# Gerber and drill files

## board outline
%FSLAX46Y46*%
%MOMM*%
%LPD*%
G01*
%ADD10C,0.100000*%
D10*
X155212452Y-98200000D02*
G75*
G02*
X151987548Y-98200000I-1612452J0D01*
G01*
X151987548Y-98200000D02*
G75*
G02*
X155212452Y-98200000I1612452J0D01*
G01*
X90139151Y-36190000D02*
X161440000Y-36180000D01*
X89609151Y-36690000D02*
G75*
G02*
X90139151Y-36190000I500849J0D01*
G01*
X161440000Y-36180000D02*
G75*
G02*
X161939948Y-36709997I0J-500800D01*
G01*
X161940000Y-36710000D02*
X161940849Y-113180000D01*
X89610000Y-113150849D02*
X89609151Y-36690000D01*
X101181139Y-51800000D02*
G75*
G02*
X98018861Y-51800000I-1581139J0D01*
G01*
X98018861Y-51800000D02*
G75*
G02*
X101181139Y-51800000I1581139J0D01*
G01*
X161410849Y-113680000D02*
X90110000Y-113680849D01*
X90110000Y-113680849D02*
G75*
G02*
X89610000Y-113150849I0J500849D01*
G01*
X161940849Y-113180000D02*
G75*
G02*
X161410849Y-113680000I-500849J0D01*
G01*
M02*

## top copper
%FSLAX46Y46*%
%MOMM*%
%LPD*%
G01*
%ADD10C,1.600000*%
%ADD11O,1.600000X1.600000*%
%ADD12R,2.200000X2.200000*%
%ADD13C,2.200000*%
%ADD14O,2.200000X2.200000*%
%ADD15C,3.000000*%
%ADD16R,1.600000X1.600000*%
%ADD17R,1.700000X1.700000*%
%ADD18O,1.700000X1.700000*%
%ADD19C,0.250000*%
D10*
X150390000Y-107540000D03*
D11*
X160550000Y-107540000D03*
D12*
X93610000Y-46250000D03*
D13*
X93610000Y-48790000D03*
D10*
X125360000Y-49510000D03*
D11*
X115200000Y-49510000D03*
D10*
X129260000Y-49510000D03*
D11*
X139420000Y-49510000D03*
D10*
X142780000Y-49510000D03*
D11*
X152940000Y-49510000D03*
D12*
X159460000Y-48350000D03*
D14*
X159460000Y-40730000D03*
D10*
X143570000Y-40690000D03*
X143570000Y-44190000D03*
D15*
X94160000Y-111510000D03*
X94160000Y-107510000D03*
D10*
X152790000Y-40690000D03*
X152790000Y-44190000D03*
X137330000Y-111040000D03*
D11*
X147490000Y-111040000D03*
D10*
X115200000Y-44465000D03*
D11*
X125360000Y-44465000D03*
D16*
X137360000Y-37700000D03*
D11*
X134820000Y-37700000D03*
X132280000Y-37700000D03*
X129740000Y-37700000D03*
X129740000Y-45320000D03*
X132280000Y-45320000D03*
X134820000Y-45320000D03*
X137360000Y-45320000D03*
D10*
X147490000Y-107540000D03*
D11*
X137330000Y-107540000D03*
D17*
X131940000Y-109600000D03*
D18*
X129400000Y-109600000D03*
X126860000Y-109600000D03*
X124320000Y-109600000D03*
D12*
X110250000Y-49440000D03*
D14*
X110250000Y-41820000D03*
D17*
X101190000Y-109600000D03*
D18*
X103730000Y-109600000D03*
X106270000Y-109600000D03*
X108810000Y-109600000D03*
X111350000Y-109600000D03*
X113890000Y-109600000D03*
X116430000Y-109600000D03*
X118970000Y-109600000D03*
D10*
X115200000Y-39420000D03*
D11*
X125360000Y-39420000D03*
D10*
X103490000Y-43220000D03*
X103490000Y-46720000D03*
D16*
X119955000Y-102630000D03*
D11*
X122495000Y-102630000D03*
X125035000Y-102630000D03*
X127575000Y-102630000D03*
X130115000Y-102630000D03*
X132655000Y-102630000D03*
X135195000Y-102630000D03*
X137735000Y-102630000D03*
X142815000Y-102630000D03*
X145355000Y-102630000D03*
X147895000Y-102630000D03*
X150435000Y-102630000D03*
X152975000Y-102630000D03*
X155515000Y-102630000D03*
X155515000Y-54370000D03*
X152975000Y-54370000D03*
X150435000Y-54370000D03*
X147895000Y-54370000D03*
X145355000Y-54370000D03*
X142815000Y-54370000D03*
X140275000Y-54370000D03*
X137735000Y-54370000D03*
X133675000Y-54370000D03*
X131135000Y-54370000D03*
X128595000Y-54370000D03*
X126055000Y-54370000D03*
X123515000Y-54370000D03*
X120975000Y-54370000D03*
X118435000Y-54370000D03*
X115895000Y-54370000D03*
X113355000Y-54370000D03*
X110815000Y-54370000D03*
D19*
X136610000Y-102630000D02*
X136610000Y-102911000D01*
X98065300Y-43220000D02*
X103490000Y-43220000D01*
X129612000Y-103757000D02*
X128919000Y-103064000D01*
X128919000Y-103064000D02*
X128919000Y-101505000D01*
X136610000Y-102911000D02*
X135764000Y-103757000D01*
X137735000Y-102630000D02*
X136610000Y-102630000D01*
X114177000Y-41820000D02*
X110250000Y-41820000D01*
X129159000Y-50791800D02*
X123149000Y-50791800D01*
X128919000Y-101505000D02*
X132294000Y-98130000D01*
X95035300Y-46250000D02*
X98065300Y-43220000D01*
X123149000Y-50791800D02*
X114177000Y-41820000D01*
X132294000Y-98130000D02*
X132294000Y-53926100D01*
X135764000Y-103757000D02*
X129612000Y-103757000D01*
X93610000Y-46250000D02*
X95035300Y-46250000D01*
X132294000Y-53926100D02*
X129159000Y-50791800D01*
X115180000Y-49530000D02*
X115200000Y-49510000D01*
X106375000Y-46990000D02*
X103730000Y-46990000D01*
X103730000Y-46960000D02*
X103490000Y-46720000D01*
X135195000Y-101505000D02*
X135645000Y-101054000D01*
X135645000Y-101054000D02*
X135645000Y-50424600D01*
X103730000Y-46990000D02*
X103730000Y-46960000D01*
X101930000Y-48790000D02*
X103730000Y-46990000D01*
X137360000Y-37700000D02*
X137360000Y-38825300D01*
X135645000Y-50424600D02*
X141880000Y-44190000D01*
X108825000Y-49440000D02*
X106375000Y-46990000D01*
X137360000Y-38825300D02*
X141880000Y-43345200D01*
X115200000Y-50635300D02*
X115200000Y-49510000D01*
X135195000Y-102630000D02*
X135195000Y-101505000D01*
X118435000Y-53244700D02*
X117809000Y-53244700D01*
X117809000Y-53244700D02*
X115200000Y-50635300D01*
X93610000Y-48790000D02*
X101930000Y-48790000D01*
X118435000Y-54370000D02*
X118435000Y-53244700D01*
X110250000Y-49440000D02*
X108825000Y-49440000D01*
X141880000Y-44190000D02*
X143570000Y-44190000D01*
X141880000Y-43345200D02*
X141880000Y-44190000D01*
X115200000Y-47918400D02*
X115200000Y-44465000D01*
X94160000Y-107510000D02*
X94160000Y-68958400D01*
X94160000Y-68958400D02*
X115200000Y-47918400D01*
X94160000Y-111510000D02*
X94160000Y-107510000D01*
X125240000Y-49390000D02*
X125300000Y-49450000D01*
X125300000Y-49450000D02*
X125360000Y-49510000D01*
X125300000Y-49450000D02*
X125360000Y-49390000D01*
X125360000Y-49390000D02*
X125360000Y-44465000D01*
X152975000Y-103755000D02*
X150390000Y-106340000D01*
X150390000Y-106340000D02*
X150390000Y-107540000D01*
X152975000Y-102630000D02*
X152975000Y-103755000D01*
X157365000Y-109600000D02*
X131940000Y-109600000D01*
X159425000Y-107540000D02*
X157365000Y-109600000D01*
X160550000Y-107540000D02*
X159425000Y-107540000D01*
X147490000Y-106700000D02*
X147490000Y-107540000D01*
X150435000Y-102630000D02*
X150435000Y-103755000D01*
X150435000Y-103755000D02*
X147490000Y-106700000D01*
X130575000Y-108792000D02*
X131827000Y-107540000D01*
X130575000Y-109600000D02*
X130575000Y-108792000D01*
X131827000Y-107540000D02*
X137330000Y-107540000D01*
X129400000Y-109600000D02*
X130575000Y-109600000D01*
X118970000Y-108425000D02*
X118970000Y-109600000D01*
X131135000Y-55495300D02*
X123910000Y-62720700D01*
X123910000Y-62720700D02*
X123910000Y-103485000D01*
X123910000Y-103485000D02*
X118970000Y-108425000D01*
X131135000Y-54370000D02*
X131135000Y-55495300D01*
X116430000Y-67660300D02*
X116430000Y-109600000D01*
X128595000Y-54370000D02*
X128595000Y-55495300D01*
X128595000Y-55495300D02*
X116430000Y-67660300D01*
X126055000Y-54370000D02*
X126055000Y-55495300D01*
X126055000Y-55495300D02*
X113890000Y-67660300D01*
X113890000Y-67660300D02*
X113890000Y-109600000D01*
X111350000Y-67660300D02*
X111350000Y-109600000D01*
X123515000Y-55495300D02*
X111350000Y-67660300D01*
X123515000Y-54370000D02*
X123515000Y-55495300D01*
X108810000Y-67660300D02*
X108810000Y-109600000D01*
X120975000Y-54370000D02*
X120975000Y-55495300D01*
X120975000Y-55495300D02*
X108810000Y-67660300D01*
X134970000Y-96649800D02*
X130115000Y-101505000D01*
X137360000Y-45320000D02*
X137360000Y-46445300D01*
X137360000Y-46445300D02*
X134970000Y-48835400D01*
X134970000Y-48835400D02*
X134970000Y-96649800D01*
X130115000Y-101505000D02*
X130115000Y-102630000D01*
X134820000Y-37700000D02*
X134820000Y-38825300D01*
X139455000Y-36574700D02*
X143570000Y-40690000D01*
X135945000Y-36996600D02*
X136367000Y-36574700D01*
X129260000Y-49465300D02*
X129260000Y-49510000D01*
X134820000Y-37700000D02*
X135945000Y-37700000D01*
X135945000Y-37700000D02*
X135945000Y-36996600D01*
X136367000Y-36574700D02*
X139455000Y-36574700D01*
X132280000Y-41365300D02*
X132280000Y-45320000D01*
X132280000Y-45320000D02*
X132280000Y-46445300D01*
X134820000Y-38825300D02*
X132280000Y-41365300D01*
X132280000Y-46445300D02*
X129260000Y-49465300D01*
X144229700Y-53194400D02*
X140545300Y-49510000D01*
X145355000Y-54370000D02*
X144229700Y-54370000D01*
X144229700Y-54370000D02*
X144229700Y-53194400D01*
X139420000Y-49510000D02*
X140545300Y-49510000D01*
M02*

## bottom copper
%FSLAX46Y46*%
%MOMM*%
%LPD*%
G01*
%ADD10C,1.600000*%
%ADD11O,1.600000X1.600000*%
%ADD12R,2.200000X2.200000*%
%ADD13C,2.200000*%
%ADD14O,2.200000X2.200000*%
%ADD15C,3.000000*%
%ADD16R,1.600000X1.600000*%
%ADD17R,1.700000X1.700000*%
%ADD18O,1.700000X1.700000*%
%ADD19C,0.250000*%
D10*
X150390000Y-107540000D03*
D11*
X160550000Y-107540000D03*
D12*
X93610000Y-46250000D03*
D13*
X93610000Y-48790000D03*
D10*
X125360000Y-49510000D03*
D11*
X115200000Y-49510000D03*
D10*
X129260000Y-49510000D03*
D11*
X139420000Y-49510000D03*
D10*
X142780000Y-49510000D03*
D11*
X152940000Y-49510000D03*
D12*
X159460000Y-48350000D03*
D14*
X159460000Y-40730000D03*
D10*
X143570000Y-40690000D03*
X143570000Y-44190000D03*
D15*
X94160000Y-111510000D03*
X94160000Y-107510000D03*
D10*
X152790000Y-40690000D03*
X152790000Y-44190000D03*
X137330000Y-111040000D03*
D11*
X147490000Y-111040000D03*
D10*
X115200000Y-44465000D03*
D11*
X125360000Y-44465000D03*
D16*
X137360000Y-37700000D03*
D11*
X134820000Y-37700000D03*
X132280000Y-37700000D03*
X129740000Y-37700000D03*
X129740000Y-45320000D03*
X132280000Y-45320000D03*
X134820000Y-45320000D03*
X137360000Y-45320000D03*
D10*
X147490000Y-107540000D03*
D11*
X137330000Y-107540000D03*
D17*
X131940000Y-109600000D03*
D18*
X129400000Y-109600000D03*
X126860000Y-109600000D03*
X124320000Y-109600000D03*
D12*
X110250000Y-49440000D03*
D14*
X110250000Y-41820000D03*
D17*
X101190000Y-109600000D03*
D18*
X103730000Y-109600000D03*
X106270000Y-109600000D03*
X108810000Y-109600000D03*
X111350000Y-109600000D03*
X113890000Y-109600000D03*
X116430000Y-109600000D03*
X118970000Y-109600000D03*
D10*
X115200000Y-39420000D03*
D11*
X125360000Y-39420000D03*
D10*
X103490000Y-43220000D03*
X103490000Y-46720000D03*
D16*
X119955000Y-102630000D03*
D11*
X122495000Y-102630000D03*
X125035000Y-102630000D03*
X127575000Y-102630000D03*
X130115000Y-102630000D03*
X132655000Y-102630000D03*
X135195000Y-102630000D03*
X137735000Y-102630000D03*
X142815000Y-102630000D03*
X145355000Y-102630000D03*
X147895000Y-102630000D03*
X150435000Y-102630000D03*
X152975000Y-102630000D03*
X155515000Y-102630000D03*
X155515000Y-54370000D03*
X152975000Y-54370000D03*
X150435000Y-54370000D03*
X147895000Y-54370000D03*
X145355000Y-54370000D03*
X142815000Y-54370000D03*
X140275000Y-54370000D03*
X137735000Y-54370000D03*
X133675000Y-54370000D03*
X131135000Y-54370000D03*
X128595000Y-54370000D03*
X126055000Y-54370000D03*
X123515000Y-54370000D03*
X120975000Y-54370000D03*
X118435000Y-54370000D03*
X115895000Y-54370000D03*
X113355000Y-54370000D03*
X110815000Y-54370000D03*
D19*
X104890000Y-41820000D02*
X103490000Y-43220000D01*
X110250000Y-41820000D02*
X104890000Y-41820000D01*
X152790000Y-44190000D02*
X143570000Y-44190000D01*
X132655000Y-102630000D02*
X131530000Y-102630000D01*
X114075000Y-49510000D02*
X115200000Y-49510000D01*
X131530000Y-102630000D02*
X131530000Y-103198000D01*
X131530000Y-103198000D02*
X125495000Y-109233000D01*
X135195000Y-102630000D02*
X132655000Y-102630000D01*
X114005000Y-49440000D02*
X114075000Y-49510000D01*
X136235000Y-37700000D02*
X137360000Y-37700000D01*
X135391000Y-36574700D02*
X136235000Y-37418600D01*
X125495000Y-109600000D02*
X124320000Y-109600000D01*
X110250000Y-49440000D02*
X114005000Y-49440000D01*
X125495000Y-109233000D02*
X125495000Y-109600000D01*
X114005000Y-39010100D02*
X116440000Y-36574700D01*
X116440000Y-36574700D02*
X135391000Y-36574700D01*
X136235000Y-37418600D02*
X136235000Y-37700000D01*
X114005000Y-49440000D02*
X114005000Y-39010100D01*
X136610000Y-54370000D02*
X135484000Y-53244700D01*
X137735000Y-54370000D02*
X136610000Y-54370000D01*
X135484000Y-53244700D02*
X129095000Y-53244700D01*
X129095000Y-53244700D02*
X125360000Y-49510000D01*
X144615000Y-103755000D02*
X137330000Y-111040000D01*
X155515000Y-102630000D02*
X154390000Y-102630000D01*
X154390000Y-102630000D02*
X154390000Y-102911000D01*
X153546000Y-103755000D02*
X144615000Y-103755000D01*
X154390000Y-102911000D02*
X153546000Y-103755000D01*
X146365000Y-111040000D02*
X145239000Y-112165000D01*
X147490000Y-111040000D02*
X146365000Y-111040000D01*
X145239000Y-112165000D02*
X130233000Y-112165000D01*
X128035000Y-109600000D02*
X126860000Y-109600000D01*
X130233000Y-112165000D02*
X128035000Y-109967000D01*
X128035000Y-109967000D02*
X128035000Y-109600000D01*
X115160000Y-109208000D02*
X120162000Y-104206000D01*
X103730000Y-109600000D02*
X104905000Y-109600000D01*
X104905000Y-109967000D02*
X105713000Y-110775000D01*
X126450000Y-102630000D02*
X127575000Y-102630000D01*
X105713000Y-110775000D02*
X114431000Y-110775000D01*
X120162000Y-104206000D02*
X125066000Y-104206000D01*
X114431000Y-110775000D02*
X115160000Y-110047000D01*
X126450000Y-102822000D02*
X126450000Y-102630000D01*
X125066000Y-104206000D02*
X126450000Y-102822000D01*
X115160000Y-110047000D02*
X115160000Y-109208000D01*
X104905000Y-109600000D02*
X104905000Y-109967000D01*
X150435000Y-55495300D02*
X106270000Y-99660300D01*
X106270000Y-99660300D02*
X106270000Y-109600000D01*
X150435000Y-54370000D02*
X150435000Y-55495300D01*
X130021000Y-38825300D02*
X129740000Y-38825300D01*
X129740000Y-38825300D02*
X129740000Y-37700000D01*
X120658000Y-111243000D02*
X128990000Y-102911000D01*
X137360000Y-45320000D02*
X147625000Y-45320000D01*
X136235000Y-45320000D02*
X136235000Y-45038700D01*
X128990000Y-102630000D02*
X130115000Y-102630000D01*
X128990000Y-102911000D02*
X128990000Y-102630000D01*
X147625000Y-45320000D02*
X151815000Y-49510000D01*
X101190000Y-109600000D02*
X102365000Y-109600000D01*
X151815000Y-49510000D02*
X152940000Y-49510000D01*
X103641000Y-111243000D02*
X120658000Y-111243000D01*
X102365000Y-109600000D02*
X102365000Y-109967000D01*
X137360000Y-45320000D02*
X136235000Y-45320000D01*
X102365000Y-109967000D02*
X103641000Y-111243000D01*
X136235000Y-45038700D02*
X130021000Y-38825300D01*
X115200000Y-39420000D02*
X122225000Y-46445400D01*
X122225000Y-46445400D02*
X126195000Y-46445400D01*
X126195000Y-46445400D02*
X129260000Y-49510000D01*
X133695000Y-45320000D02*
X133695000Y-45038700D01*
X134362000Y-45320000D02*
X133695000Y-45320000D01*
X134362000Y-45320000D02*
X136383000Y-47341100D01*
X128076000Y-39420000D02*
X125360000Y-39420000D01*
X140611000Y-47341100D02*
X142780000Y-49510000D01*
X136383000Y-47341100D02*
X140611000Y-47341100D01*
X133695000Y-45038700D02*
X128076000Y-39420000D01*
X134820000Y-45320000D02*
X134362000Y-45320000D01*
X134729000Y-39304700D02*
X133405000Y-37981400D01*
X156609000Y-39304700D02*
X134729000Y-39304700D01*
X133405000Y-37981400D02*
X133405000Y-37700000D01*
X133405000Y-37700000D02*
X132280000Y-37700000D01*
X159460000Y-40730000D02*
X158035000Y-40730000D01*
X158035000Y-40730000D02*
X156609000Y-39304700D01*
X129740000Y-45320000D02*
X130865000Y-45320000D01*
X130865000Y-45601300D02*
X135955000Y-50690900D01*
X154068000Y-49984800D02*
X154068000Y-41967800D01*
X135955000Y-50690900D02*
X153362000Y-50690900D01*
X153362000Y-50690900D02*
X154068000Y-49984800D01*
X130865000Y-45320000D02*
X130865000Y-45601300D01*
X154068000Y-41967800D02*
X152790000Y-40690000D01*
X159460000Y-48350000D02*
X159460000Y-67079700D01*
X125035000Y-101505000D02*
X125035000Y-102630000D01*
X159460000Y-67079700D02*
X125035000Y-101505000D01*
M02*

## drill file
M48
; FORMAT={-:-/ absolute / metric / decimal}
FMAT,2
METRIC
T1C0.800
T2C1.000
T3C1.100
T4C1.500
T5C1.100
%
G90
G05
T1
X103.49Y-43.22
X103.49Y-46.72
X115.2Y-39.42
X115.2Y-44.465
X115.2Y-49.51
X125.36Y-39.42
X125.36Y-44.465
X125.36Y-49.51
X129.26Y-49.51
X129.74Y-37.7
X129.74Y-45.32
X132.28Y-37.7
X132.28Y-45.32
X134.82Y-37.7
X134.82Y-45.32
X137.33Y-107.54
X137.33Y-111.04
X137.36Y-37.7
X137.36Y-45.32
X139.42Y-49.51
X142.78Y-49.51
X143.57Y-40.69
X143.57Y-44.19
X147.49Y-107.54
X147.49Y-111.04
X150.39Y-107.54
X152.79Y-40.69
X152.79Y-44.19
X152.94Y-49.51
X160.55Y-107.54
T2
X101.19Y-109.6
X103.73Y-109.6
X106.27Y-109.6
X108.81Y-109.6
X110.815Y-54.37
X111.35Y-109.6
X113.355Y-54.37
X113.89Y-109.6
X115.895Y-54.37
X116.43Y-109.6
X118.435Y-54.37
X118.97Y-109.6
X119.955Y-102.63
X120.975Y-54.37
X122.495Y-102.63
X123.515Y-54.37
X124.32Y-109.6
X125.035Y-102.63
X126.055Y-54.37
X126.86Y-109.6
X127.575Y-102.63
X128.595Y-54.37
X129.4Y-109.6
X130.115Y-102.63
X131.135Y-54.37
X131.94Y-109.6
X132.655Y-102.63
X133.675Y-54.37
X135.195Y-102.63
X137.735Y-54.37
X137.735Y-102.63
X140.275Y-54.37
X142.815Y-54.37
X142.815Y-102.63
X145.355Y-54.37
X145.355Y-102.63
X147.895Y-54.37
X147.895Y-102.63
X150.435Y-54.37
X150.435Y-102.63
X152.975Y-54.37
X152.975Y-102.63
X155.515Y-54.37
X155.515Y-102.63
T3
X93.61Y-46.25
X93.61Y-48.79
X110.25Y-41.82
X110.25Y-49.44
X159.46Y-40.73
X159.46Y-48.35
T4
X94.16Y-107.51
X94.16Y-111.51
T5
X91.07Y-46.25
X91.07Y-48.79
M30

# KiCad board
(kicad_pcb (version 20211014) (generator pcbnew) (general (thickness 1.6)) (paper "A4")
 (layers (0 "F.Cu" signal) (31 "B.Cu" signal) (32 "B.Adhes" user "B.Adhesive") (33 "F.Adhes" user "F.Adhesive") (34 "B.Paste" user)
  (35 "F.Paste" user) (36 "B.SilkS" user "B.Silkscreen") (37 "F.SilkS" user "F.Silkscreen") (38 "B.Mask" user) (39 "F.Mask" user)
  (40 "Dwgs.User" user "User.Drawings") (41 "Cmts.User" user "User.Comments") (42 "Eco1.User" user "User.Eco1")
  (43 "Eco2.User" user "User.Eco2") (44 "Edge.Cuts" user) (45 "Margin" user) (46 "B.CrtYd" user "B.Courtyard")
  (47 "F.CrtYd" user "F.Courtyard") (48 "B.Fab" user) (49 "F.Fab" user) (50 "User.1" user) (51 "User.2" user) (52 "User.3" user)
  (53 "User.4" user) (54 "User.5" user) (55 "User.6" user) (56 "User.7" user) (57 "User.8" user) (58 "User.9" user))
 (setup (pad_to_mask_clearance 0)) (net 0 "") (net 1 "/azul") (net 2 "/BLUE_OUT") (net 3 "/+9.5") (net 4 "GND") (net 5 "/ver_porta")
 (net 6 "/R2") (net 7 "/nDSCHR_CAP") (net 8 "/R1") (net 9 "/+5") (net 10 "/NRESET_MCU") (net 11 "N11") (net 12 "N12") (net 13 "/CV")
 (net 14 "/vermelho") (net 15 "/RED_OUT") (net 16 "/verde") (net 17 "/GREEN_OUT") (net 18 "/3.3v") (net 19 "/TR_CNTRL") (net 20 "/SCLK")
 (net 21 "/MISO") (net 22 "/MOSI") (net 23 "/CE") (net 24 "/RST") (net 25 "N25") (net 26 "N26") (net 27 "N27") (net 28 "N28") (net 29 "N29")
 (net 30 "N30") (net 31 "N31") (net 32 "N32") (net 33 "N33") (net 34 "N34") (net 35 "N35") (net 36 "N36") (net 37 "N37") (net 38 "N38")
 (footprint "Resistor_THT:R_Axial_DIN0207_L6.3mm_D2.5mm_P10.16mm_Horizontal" (layer "F.Cu") (at 150.39 107.54)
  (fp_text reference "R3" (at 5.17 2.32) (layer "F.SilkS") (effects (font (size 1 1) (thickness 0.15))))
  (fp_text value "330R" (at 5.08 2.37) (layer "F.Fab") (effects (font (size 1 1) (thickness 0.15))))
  (pad "1" thru_hole circle (at 0 0) (size 1.6 1.6) (drill 0.8) (layers *.Cu *.Mask) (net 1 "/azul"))
  (pad "2" thru_hole oval (at 10.16 0) (size 1.6 1.6) (drill 0.8) (layers *.Cu *.Mask) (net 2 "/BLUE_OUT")))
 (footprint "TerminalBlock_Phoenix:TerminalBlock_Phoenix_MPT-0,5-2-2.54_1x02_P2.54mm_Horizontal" (layer "F.Cu") (at 93.61 46.25 -90)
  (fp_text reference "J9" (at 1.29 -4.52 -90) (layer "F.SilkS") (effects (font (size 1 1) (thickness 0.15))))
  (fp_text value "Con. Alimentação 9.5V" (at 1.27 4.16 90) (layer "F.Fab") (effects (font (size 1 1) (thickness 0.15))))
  (pad "" np_thru_hole circle (at 2.54 2.54 270) (size 1.1 1.1) (drill 1.1) (layers *.Cu *.Mask))
  (pad "" np_thru_hole circle (at 0 2.54 270) (size 1.1 1.1) (drill 1.1) (layers *.Cu *.Mask))
  (pad "1" thru_hole rect (at 0 0 270) (size 2.2 2.2) (drill 1.1) (layers *.Cu *.Mask) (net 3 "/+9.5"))
  (pad "2" thru_hole circle (at 2.54 0 270) (size 2.2 2.2) (drill 1.1) (layers *.Cu *.Mask) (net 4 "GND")))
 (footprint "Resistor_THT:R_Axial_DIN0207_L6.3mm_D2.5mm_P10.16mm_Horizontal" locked (layer "F.Cu") (at 125.36 49.51 180)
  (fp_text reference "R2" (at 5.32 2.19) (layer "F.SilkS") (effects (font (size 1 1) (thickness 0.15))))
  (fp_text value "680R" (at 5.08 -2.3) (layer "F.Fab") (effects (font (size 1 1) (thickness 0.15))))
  (pad "1" thru_hole circle locked (at 0 0 180) (size 1.6 1.6) (drill 0.8) (layers *.Cu *.Mask) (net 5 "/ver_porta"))
  (pad "2" thru_hole oval locked (at 10.16 0 180) (size 1.6 1.6) (drill 0.8) (layers *.Cu *.Mask) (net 4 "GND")))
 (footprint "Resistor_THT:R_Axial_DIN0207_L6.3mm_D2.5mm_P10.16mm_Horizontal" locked (layer "F.Cu") (at 129.26 49.51)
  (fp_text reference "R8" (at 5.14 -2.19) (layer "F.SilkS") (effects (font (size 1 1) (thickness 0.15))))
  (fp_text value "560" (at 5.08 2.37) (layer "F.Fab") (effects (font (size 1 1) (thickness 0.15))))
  (pad "1" thru_hole circle locked (at 0 0) (size 1.6 1.6) (drill 0.8) (layers *.Cu *.Mask) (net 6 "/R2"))
  (pad "2" thru_hole oval locked (at 10.16 0) (size 1.6 1.6) (drill 0.8) (layers *.Cu *.Mask) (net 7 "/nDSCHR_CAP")))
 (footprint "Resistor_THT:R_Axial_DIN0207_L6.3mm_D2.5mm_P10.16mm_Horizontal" (layer "F.Cu") (at 142.78 49.51)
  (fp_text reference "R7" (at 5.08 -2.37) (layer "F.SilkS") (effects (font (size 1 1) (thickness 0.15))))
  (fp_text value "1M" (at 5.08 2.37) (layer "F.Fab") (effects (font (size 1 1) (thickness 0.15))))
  (pad "1" thru_hole circle (at 0 0) (size 1.6 1.6) (drill 0.8) (layers *.Cu *.Mask) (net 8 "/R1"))
  (pad "2" thru_hole oval (at 10.16 0) (size 1.6 1.6) (drill 0.8) (layers *.Cu *.Mask) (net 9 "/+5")))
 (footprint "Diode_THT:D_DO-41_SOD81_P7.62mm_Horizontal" (layer "F.Cu") (at 159.46 48.35 90)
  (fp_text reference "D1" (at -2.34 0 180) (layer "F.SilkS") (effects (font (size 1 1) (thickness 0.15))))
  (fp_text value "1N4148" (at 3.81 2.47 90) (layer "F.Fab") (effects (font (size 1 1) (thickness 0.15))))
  (pad "1" thru_hole rect (at 0 0 90) (size 2.2 2.2) (drill 1.1) (layers *.Cu *.Mask) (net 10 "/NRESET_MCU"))
  (pad "2" thru_hole oval (at 7.62 0 90) (size 2.2 2.2) (drill 1.1) (layers *.Cu *.Mask) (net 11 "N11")))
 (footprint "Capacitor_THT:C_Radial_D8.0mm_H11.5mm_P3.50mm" (layer "F.Cu") (at 143.57 40.69 -90)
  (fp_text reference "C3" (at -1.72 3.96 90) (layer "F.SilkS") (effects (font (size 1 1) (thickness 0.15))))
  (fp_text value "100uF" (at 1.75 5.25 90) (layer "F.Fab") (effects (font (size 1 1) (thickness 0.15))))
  (pad "1" thru_hole circle (at 0 0 270) (size 1.6 1.6) (drill 0.8) (layers *.Cu *.Mask) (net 6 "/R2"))
  (pad "2" thru_hole circle (at 3.5 0 270) (size 1.6 1.6) (drill 0.8) (layers *.Cu *.Mask) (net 4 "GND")))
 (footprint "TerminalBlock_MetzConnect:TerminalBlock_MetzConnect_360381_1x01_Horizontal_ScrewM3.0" (layer "F.Cu") (at 94.16 111.51 90)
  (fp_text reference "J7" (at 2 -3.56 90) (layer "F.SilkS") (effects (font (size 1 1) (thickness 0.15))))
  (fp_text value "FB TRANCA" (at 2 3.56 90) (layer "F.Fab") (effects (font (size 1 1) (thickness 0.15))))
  (pad "1" thru_hole circle (at 0 0 90) (size 3 3) (drill 1.5) (layers *.Cu *.Mask) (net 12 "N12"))
  (pad "1" thru_hole circle (at 4 0 90) (size 3 3) (drill 1.5) (layers *.Cu *.Mask) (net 12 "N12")))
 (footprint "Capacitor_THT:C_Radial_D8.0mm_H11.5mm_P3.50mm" (layer "F.Cu") (at 152.79 40.69 -90)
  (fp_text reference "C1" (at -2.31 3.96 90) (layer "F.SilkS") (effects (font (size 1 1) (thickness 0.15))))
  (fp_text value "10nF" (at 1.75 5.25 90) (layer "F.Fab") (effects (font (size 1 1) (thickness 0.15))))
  (pad "1" thru_hole circle (at 0 0 270) (size 1.6 1.6) (drill 0.8) (layers *.Cu *.Mask) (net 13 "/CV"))
  (pad "2" thru_hole circle (at 3.5 0 270) (size 1.6 1.6) (drill 0.8) (layers *.Cu *.Mask) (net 4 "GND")))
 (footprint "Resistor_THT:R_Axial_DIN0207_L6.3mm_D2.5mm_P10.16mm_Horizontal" (layer "F.Cu") (at 137.33 111.04)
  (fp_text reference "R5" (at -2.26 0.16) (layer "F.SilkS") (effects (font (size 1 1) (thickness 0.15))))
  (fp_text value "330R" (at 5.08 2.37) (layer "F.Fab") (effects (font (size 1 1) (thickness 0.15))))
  (pad "1" thru_hole circle (at 0 0) (size 1.6 1.6) (drill 0.8) (layers *.Cu *.Mask) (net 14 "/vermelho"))
  (pad "2" thru_hole oval (at 10.16 0) (size 1.6 1.6) (drill 0.8) (layers *.Cu *.Mask) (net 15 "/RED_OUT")))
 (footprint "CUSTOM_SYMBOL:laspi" (layer "F.Cu") (at 94.1 40.08)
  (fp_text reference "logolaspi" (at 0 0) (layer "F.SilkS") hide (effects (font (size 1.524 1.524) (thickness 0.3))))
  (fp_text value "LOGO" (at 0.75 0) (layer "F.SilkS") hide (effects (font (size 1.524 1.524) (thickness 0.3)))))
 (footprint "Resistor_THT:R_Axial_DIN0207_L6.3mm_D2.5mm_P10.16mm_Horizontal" (layer "F.Cu") (at 115.2 44.465)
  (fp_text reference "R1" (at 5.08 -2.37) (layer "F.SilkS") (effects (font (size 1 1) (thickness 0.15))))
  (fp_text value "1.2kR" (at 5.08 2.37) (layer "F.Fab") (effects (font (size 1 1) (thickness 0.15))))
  (pad "1" thru_hole circle (at 0 0) (size 1.6 1.6) (drill 0.8) (layers *.Cu *.Mask) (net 12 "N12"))
  (pad "2" thru_hole oval (at 10.16 0) (size 1.6 1.6) (drill 0.8) (layers *.Cu *.Mask) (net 5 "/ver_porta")))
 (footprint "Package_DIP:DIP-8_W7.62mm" (layer "F.Cu") (at 137.36 37.7 -90)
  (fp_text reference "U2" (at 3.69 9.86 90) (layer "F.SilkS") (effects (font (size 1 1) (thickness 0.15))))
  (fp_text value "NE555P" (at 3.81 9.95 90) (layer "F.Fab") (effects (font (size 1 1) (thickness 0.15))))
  (pad "1" thru_hole rect (at 0 0 270) (size 1.6 1.6) (drill 0.8) (layers *.Cu *.Mask) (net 4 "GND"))
  (pad "2" thru_hole oval (at 0 2.54 270) (size 1.6 1.6) (drill 0.8) (layers *.Cu *.Mask) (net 6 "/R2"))
  (pad "3" thru_hole oval (at 0 5.08 270) (size 1.6 1.6) (drill 0.8) (layers *.Cu *.Mask) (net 11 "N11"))
  (pad "4" thru_hole oval (at 0 7.62 270) (size 1.6 1.6) (drill 0.8) (layers *.Cu *.Mask) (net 9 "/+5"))
  (pad "5" thru_hole oval (at 7.62 7.62 270) (size 1.6 1.6) (drill 0.8) (layers *.Cu *.Mask) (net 13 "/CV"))
  (pad "6" thru_hole oval (at 7.62 5.08 270) (size 1.6 1.6) (drill 0.8) (layers *.Cu *.Mask) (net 6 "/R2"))
  (pad "7" thru_hole oval (at 7.62 2.54 270) (size 1.6 1.6) (drill 0.8) (layers *.Cu *.Mask) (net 8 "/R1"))
  (pad "8" thru_hole oval (at 7.62 0 270) (size 1.6 1.6) (drill 0.8) (layers *.Cu *.Mask) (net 9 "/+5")))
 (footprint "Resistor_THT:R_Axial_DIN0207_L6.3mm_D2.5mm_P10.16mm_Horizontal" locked (layer "F.Cu") (at 147.49 107.54 180)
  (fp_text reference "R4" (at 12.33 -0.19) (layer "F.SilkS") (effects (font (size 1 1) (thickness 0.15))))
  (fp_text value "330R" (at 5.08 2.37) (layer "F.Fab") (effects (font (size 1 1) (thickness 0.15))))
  (pad "1" thru_hole circle locked (at 0 0 180) (size 1.6 1.6) (drill 0.8) (layers *.Cu *.Mask) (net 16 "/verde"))
  (pad "2" thru_hole oval locked (at 10.16 0 180) (size 1.6 1.6) (drill 0.8) (layers *.Cu *.Mask) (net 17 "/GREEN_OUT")))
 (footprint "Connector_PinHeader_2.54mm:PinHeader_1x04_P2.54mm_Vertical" (layer "F.Cu") (at 131.94 109.6 -90)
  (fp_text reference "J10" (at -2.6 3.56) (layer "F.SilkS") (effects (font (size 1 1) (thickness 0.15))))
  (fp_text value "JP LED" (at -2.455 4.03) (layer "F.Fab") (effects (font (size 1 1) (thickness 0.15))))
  (pad "1" thru_hole rect (at 0 0 270) (size 1.7 1.7) (drill 1) (layers *.Cu *.Mask) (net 2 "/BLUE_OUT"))
  (pad "2" thru_hole oval (at 0 2.54 270) (size 1.7 1.7) (drill 1) (layers *.Cu *.Mask) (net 17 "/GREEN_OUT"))
  (pad "3" thru_hole oval (at 0 5.08 270) (size 1.7 1.7) (drill 1) (layers *.Cu *.Mask) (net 15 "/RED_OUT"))
  (pad "4" thru_hole oval (at 0 7.62 270) (size 1.7 1.7) (drill 1) (layers *.Cu *.Mask) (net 4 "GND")))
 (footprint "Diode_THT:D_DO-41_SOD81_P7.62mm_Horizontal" (layer "F.Cu") (at 110.25 49.44 90)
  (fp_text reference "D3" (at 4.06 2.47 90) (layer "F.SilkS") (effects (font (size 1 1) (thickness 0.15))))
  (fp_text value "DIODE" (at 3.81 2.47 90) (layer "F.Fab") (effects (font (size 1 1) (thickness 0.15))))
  (pad "1" thru_hole rect (at 0 0 90) (size 2.2 2.2) (drill 1.1) (layers *.Cu *.Mask) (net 4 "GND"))
  (pad "2" thru_hole oval (at 7.62 0 90) (size 2.2 2.2) (drill 1.1) (layers *.Cu *.Mask) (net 3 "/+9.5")))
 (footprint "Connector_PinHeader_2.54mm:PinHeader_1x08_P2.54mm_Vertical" (layer "F.Cu") (at 101.19 109.6 90)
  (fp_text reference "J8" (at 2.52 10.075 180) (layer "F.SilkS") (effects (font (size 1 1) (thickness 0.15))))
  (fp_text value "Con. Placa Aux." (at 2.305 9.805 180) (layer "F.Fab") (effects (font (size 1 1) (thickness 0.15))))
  (pad "1" thru_hole rect (at 0 0 90) (size 1.7 1.7) (drill 1) (layers *.Cu *.Mask) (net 9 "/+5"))
  (pad "2" thru_hole oval (at 0 2.54 90) (size 1.7 1.7) (drill 1) (layers *.Cu *.Mask) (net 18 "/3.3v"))
  (pad "3" thru_hole oval (at 0 5.08 90) (size 1.7 1.7) (drill 1) (layers *.Cu *.Mask) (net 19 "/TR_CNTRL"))
  (pad "4" thru_hole oval (at 0 7.62 90) (size 1.7 1.7) (drill 1) (layers *.Cu *.Mask) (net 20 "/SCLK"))
  (pad "5" thru_hole oval (at 0 10.16 90) (size 1.7 1.7) (drill 1) (layers *.Cu *.Mask) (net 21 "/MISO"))
  (pad "6" thru_hole oval (at 0 12.7 90) (size 1.7 1.7) (drill 1) (layers *.Cu *.Mask) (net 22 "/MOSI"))
  (pad "7" thru_hole oval (at 0 15.24 90) (size 1.7 1.7) (drill 1) (layers *.Cu *.Mask) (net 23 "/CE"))
  (pad "8" thru_hole oval (at 0 17.78 90) (size 1.7 1.7) (drill 1) (layers *.Cu *.Mask) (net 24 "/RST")))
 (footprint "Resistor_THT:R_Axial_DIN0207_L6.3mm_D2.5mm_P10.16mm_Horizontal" (layer "F.Cu") (at 115.2 39.42)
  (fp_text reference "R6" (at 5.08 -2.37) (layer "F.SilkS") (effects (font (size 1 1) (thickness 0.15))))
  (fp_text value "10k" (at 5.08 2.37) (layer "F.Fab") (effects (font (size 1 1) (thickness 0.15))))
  (pad "1" thru_hole circle (at 0 0) (size 1.6 1.6) (drill 0.8) (layers *.Cu *.Mask) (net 6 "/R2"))
  (pad "2" thru_hole oval (at 10.16 0) (size 1.6 1.6) (drill 0.8) (layers *.Cu *.Mask) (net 8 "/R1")))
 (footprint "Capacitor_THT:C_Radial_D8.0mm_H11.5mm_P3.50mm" (layer "F.Cu") (at 103.49 43.22 -90)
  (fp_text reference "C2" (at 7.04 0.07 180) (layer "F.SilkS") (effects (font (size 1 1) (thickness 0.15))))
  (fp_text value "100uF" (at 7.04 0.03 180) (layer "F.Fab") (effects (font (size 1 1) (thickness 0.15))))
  (pad "1" thru_hole circle (at 0 0 270) (size 1.6 1.6) (drill 0.8) (layers *.Cu *.Mask) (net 3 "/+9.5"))
  (pad "2" thru_hole circle (at 3.5 0 270) (size 1.6 1.6) (drill 0.8) (layers *.Cu *.Mask) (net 4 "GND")))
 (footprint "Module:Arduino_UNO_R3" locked (layer "B.Cu") (at 119.955 102.63)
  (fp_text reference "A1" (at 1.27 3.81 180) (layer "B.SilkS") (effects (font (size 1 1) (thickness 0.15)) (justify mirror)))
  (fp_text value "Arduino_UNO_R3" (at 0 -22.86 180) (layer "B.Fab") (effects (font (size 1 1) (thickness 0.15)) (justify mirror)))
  (pad "1" thru_hole rect locked (at 0 0 270) (size 1.6 1.6) (drill 1) (layers *.Cu *.Mask) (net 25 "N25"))
  (pad "2" thru_hole oval locked (at 2.54 0 270) (size 1.6 1.6) (drill 1) (layers *.Cu *.Mask) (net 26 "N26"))
  (pad "3" thru_hole oval locked (at 5.08 0 270) (size 1.6 1.6) (drill 1) (layers *.Cu *.Mask) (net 10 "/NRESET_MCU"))
  (pad "4" thru_hole oval locked (at 7.62 0 270) (size 1.6 1.6) (drill 1) (layers *.Cu *.Mask) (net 18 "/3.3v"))
  (pad "5" thru_hole oval locked (at 10.16 0 270) (size 1.6 1.6) (drill 1) (layers *.Cu *.Mask) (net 9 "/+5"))
  (pad "6" thru_hole oval locked (at 12.7 0 270) (size 1.6 1.6) (drill 1) (layers *.Cu *.Mask) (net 4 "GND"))
  (pad "7" thru_hole oval locked (at 15.24 0 270) (size 1.6 1.6) (drill 1) (layers *.Cu *.Mask) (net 4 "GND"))
  (pad "8" thru_hole oval locked (at 17.78 0 270) (size 1.6 1.6) (drill 1) (layers *.Cu *.Mask) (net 3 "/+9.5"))
  (pad "9" thru_hole oval locked (at 22.86 0 270) (size 1.6 1.6) (drill 1) (layers *.Cu *.Mask) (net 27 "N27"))
  (pad "10" thru_hole oval locked (at 25.4 0 270) (size 1.6 1.6) (drill 1) (layers *.Cu *.Mask) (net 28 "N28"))
  (pad "11" thru_hole oval locked (at 27.94 0 270) (size 1.6 1.6) (drill 1) (layers *.Cu *.Mask) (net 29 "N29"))
  (pad "12" thru_hole oval locked (at 30.48 0 270) (size 1.6 1.6) (drill 1) (layers *.Cu *.Mask) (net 16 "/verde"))
  (pad "13" thru_hole oval locked (at 33.02 0 270) (size 1.6 1.6) (drill 1) (layers *.Cu *.Mask) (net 1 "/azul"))
  (pad "14" thru_hole oval locked (at 35.56 0 270) (size 1.6 1.6) (drill 1) (layers *.Cu *.Mask) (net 14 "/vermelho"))
  (pad "15" thru_hole oval locked (at 35.56 -48.26 270) (size 1.6 1.6) (drill 1) (layers *.Cu *.Mask) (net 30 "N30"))
  (pad "16" thru_hole oval locked (at 33.02 -48.26 270) (size 1.6 1.6) (drill 1) (layers *.Cu *.Mask) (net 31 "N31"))
  (pad "17" thru_hole oval locked (at 30.48 -48.26 270) (size 1.6 1.6) (drill 1) (layers *.Cu *.Mask) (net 19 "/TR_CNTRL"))
  (pad "18" thru_hole oval locked (at 27.94 -48.26 270) (size 1.6 1.6) (drill 1) (layers *.Cu *.Mask) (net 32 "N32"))
  (pad "19" thru_hole oval locked (at 25.4 -48.26 270) (size 1.6 1.6) (drill 1) (layers *.Cu *.Mask) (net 7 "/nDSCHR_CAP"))
  (pad "20" thru_hole oval locked (at 22.86 -48.26 270) (size 1.6 1.6) (drill 1) (layers *.Cu *.Mask) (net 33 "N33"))
  (pad "21" thru_hole oval locked (at 20.32 -48.26 270) (size 1.6 1.6) (drill 1) (layers *.Cu *.Mask) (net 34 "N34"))
  (pad "22" thru_hole oval locked (at 17.78 -48.26 270) (size 1.6 1.6) (drill 1) (layers *.Cu *.Mask) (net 5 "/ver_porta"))
  (pad "23" thru_hole oval locked (at 13.72 -48.26 270) (size 1.6 1.6) (drill 1) (layers *.Cu *.Mask) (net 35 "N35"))
  (pad "24" thru_hole oval locked (at 11.18 -48.26 270) (size 1.6 1.6) (drill 1) (layers *.Cu *.Mask) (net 24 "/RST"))
  (pad "25" thru_hole oval locked (at 8.64 -48.26 270) (size 1.6 1.6) (drill 1) (layers *.Cu *.Mask) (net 23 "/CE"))
  (pad "26" thru_hole oval locked (at 6.1 -48.26 270) (size 1.6 1.6) (drill 1) (layers *.Cu *.Mask) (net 22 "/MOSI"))
  (pad "27" thru_hole oval locked (at 3.56 -48.26 270) (size 1.6 1.6) (drill 1) (layers *.Cu *.Mask) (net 21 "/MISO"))
  (pad "28" thru_hole oval locked (at 1.02 -48.26 270) (size 1.6 1.6) (drill 1) (layers *.Cu *.Mask) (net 20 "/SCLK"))
  (pad "29" thru_hole oval locked (at -1.52 -48.26 270) (size 1.6 1.6) (drill 1) (layers *.Cu *.Mask) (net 4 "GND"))
  (pad "30" thru_hole oval locked (at -4.06 -48.26 270) (size 1.6 1.6) (drill 1) (layers *.Cu *.Mask) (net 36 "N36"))
  (pad "31" thru_hole oval locked (at -6.6 -48.26 270) (size 1.6 1.6) (drill 1) (layers *.Cu *.Mask) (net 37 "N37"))
  (pad "32" thru_hole oval locked (at -9.14 -48.26 270) (size 1.6 1.6) (drill 1) (layers *.Cu *.Mask) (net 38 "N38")))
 (gr_circle locked (center 153.6 98.2) (end 152.8 96.8) (layer "Edge.Cuts") (width 0.1) (fill none))
 (gr_line (start 90.139151 36.19) (end 161.44 36.18) (layer "Edge.Cuts") (width 0.1))
 (gr_arc (start 89.609151 36.69) (mid 89.766307 36.325686) (end 90.139151 36.19) (layer "Edge.Cuts") (width 0.1))
 (gr_arc (start 161.44 36.18) (mid 161.804314 36.337156) (end 161.94 36.71) (layer "Edge.Cuts") (width 0.1))
 (gr_line (start 161.94 36.71) (end 161.940849 113.18) (layer "Edge.Cuts") (width 0.1))
 (gr_line (start 89.61 113.150849) (end 89.609151 36.69) (layer "Edge.Cuts") (width 0.1))
 (gr_circle (center 99.6 51.8) (end 99.1 50.3) (layer "Edge.Cuts") (width 0.1) (fill none))
 (gr_line (start 161.410849 113.68) (end 90.11 113.680849) (layer "Edge.Cuts") (width 0.1))
 (gr_arc (start 90.11 113.680849) (mid 89.745686 113.523693) (end 89.61 113.150849) (layer "Edge.Cuts") (width 0.1))
 (gr_arc (start 161.940849 113.18) (mid 161.783693 113.544314) (end 161.410849 113.68) (layer "Edge.Cuts") (width 0.1))
 (segment (start 136.61 102.63) (end 136.61 102.911) (width 0.25) (layer "F.Cu") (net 3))
 (segment (start 98.0653 43.22) (end 103.49 43.22) (width 0.25) (layer "F.Cu") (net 3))
 (segment (start 129.612 103.757) (end 128.919 103.064) (width 0.25) (layer "F.Cu") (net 3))
 (segment (start 128.919 103.064) (end 128.919 101.505) (width 0.25) (layer "F.Cu") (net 3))
 (segment (start 136.61 102.911) (end 135.764 103.757) (width 0.25) (layer "F.Cu") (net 3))
 (segment (start 137.735 102.63) (end 136.61 102.63) (width 0.25) (layer "F.Cu") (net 3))
 (segment (start 114.177 41.82) (end 110.25 41.82) (width 0.25) (layer "F.Cu") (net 3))
 (segment (start 129.159 50.7918) (end 123.149 50.7918) (width 0.25) (layer "F.Cu") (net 3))
 (segment (start 128.919 101.505) (end 132.294 98.13) (width 0.25) (layer "F.Cu") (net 3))
 (segment (start 95.0353 46.25) (end 98.0653 43.22) (width 0.25) (layer "F.Cu") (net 3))
 (segment (start 123.149 50.7918) (end 114.177 41.82) (width 0.25) (layer "F.Cu") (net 3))
 (segment (start 132.294 98.13) (end 132.294 53.9261) (width 0.25) (layer "F.Cu") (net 3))
 (segment (start 135.764 103.757) (end 129.612 103.757) (width 0.25) (layer "F.Cu") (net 3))
 (segment (start 93.61 46.25) (end 95.0353 46.25) (width 0.25) (layer "F.Cu") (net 3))
 (segment (start 132.294 53.9261) (end 129.159 50.7918) (width 0.25) (layer "F.Cu") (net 3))
 (segment (start 104.89 41.82) (end 103.49 43.22) (width 0.25) (layer "B.Cu") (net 3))
 (segment (start 110.25 41.82) (end 104.89 41.82) (width 0.25) (layer "B.Cu") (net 3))
 (segment (start 115.18 49.53) (end 115.2 49.51) (width 0.25) (layer "F.Cu") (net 4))
 (segment (start 106.375 46.99) (end 103.73 46.99) (width 0.25) (layer "F.Cu") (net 4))
 (segment (start 103.73 46.96) (end 103.49 46.72) (width 0.25) (layer "F.Cu") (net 4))
 (segment (start 135.195 101.505) (end 135.645 101.054) (width 0.25) (layer "F.Cu") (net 4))
 (segment (start 135.645 101.054) (end 135.645 50.4246) (width 0.25) (layer "F.Cu") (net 4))
 (segment (start 103.73 46.99) (end 103.73 46.96) (width 0.25) (layer "F.Cu") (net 4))
 (segment (start 101.93 48.79) (end 103.73 46.99) (width 0.25) (layer "F.Cu") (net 4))
 (segment (start 137.36 37.7) (end 137.36 38.8253) (width 0.25) (layer "F.Cu") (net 4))
 (segment (start 135.645 50.4246) (end 141.88 44.19) (width 0.25) (layer "F.Cu") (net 4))
 (segment (start 108.825 49.44) (end 106.375 46.99) (width 0.25) (layer "F.Cu") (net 4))
 (segment (start 137.36 38.8253) (end 141.88 43.3452) (width 0.25) (layer "F.Cu") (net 4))
 (segment (start 115.2 50.6353) (end 115.2 49.51) (width 0.25) (layer "F.Cu") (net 4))
 (segment (start 135.195 102.63) (end 135.195 101.505) (width 0.25) (layer "F.Cu") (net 4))
 (segment (start 118.435 53.2447) (end 117.809 53.2447) (width 0.25) (layer "F.Cu") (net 4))
 (segment (start 117.809 53.2447) (end 115.2 50.6353) (width 0.25) (layer "F.Cu") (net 4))
 (segment (start 93.61 48.79) (end 101.93 48.79) (width 0.25) (layer "F.Cu") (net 4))
 (segment (start 118.435 54.37) (end 118.435 53.2447) (width 0.25) (layer "F.Cu") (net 4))
 (segment (start 110.25 49.44) (end 108.825 49.44) (width 0.25) (layer "F.Cu") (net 4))
 (segment (start 141.88 44.19) (end 143.57 44.19) (width 0.25) (layer "F.Cu") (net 4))
 (segment (start 141.88 43.3452) (end 141.88 44.19) (width 0.25) (layer "F.Cu") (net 4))
 (segment (start 152.79 44.19) (end 143.57 44.19) (width 0.25) (layer "B.Cu") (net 4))
 (segment (start 132.655 102.63) (end 131.53 102.63) (width 0.25) (layer "B.Cu") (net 4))
 (segment (start 114.075 49.51) (end 115.2 49.51) (width 0.25) (layer "B.Cu") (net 4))
 (segment (start 131.53 102.63) (end 131.53 103.198) (width 0.25) (layer "B.Cu") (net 4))
 (segment (start 131.53 103.198) (end 125.495 109.233) (width 0.25) (layer "B.Cu") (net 4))
 (segment (start 135.195 102.63) (end 132.655 102.63) (width 0.25) (layer "B.Cu") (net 4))
 (segment (start 114.005 49.44) (end 114.075 49.51) (width 0.25) (layer "B.Cu") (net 4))
 (segment (start 136.235 37.7) (end 137.36 37.7) (width 0.25) (layer "B.Cu") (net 4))
 (segment (start 135.391 36.5747) (end 136.235 37.4186) (width 0.25) (layer "B.Cu") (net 4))
 (segment (start 125.495 109.6) (end 124.32 109.6) (width 0.25) (layer "B.Cu") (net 4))
 (segment (start 110.25 49.44) (end 114.005 49.44) (width 0.25) (layer "B.Cu") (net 4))
 (segment (start 125.495 109.233) (end 125.495 109.6) (width 0.25) (layer "B.Cu") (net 4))
 (segment (start 114.005 39.0101) (end 116.44 36.5747) (width 0.25) (layer "B.Cu") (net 4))
 (segment (start 116.44 36.5747) (end 135.391 36.5747) (width 0.25) (layer "B.Cu") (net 4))
 (segment (start 136.235 37.4186) (end 136.235 37.7) (width 0.25) (layer "B.Cu") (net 4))
 (segment (start 114.005 49.44) (end 114.005 39.0101) (width 0.25) (layer "B.Cu") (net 4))
 (segment (start 115.2 47.9184) (end 115.2 44.465) (width 0.25) (layer "F.Cu") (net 12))
 (segment (start 94.16 107.51) (end 94.16 68.9584) (width 0.25) (layer "F.Cu") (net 12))
 (segment (start 94.16 68.9584) (end 115.2 47.9184) (width 0.25) (layer "F.Cu") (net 12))
 (segment (start 94.16 111.51) (end 94.16 107.51) (width 0.25) (layer "F.Cu") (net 12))
 (segment (start 125.24 49.39) (end 125.3 49.45) (width 0.25) (layer "F.Cu") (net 5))
 (segment (start 125.3 49.45) (end 125.36 49.51) (width 0.25) (layer "F.Cu") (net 5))
 (segment (start 125.3 49.45) (end 125.36 49.39) (width 0.25) (layer "F.Cu") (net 5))
 (segment (start 125.36 49.39) (end 125.36 44.465) (width 0.25) (layer "F.Cu") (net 5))
 (segment (start 136.61 54.37) (end 135.484 53.2447) (width 0.25) (layer "B.Cu") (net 5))
 (segment (start 137.735 54.37) (end 136.61 54.37) (width 0.25) (layer "B.Cu") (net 5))
 (segment (start 135.484 53.2447) (end 129.095 53.2447) (width 0.25) (layer "B.Cu") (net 5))
 (segment (start 129.095 53.2447) (end 125.36 49.51) (width 0.25) (layer "B.Cu") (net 5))
 (segment (start 152.975 103.755) (end 150.39 106.34) (width 0.25) (layer "F.Cu") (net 1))
 (segment (start 150.39 106.34) (end 150.39 107.54) (width 0.25) (layer "F.Cu") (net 1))
 (segment (start 152.975 102.63) (end 152.975 103.755) (width 0.25) (layer "F.Cu") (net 1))
 (segment (start 157.365 109.6) (end 131.94 109.6) (width 0.25) (layer "F.Cu") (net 2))
 (segment (start 159.425 107.54) (end 157.365 109.6) (width 0.25) (layer "F.Cu") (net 2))
 (segment (start 160.55 107.54) (end 159.425 107.54) (width 0.25) (layer "F.Cu") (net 2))
 (segment (start 147.49 106.7) (end 147.49 107.54) (width 0.25) (layer "F.Cu") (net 16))
 (segment (start 150.435 102.63) (end 150.435 103.755) (width 0.25) (layer "F.Cu") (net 16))
 (segment (start 150.435 103.755) (end 147.49 106.7) (width 0.25) (layer "F.Cu") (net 16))
 (segment (start 130.575 108.792) (end 131.827 107.54) (width 0.25) (layer "F.Cu") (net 17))
 (segment (start 130.575 109.6) (end 130.575 108.792) (width 0.25) (layer "F.Cu") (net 17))
 (segment (start 131.827 107.54) (end 137.33 107.54) (width 0.25) (layer "F.Cu") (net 17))
 (segment (start 129.4 109.6) (end 130.575 109.6) (width 0.25) (layer "F.Cu") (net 17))
 (segment (start 144.615 103.755) (end 137.33 111.04) (width 0.25) (layer "B.Cu") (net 14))
 (segment (start 155.515 102.63) (end 154.39 102.63) (width 0.25) (layer "B.Cu") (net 14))
 (segment (start 154.39 102.63) (end 154.39 102.911) (width 0.25) (layer "B.Cu") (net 14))
 (segment (start 153.546 103.755) (end 144.615 103.755) (width 0.25) (layer "B.Cu") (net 14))
 (segment (start 154.39 102.911) (end 153.546 103.755) (width 0.25) (layer "B.Cu") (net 14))
 (segment (start 146.365 111.04) (end 145.239 112.165) (width 0.25) (layer "B.Cu") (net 15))
 (segment (start 147.49 111.04) (end 146.365 111.04) (width 0.25) (layer "B.Cu") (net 15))
 (segment (start 145.239 112.165) (end 130.233 112.165) (width 0.25) (layer "B.Cu") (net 15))
 (segment (start 128.035 109.6) (end 126.86 109.6) (width 0.25) (layer "B.Cu") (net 15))
 (segment (start 130.233 112.165) (end 128.035 109.967) (width 0.25) (layer "B.Cu") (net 15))
 (segment (start 128.035 109.967) (end 128.035 109.6) (width 0.25) (layer "B.Cu") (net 15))
 (segment (start 115.16 109.208) (end 120.162 104.206) (width 0.25) (layer "B.Cu") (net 18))
 (segment (start 103.73 109.6) (end 104.905 109.6) (width 0.25) (layer "B.Cu") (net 18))
 (segment (start 104.905 109.967) (end 105.713 110.775) (width 0.25) (layer "B.Cu") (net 18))
 (segment (start 126.45 102.63) (end 127.575 102.63) (width 0.25) (layer "B.Cu") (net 18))
 (segment (start 105.713 110.775) (end 114.431 110.775) (width 0.25) (layer "B.Cu") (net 18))
 (segment (start 120.162 104.206) (end 125.066 104.206) (width 0.25) (layer "B.Cu") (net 18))
 (segment (start 114.431 110.775) (end 115.16 110.047) (width 0.25) (layer "B.Cu") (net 18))
 (segment (start 126.45 102.822) (end 126.45 102.63) (width 0.25) (layer "B.Cu") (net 18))
 (segment (start 125.066 104.206) (end 126.45 102.822) (width 0.25) (layer "B.Cu") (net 18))
 (segment (start 115.16 110.047) (end 115.16 109.208) (width 0.25) (layer "B.Cu") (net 18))
 (segment (start 104.905 109.6) (end 104.905 109.967) (width 0.25) (layer "B.Cu") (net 18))
 (segment (start 118.97 108.425) (end 118.97 109.6) (width 0.25) (layer "F.Cu") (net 24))
 (segment (start 131.135 55.4953) (end 123.91 62.7207) (width 0.25) (layer "F.Cu") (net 24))
 (segment (start 123.91 62.7207) (end 123.91 103.485) (width 0.25) (layer "F.Cu") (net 24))
 (segment (start 123.91 103.485) (end 118.97 108.425) (width 0.25) (layer "F.Cu") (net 24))
 (segment (start 131.135 54.37) (end 131.135 55.4953) (width 0.25) (layer "F.Cu") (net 24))
 (segment (start 150.435 55.4953) (end 106.27 99.6603) (width 0.25) (layer "B.Cu") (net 19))
 (segment (start 106.27 99.6603) (end 106.27 109.6) (width 0.25) (layer "B.Cu") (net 19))
 (segment (start 150.435 54.37) (end 150.435 55.4953) (width 0.25) (layer "B.Cu") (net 19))
 (segment (start 116.43 67.6603) (end 116.43 109.6) (width 0.25) (layer "F.Cu") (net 23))
 (segment (start 128.595 54.37) (end 128.595 55.4953) (width 0.25) (layer "F.Cu") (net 23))
 (segment (start 128.595 55.4953) (end 116.43 67.6603) (width 0.25) (layer "F.Cu") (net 23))
 (segment (start 126.055 54.37) (end 126.055 55.4953) (width 0.25) (layer "F.Cu") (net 22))
 (segment (start 126.055 55.4953) (end 113.89 67.6603) (width 0.25) (layer "F.Cu") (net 22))
 (segment (start 113.89 67.6603) (end 113.89 109.6) (width 0.25) (layer "F.Cu") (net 22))
 (segment (start 111.35 67.6603) (end 111.35 109.6) (width 0.25) (layer "F.Cu") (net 21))
 (segment (start 123.515 55.4953) (end 111.35 67.6603) (width 0.25) (layer "F.Cu") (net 21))
 (segment (start 123.515 54.37) (end 123.515 55.4953) (width 0.25) (layer "F.Cu") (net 21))
 (segment (start 108.81 67.6603) (end 108.81 109.6) (width 0.25) (layer "F.Cu") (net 20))
 (segment (start 120.975 54.37) (end 120.975 55.4953) (width 0.25) (layer "F.Cu") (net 20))
 (segment (start 120.975 55.4953) (end 108.81 67.6603) (width 0.25) (layer "F.Cu") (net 20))
 (segment (start 134.97 96.6498) (end 130.115 101.505) (width 0.25) (layer "F.Cu") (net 9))
 (segment (start 137.36 45.32) (end 137.36 46.4453) (width 0.25) (layer "F.Cu") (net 9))
 (segment (start 137.36 46.4453) (end 134.97 48.8354) (width 0.25) (layer "F.Cu") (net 9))
 (segment (start 134.97 48.8354) (end 134.97 96.6498) (width 0.25) (layer "F.Cu") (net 9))
 (segment (start 130.115 101.505) (end 130.115 102.63) (width 0.25) (layer "F.Cu") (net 9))
 (segment (start 130.021 38.8253) (end 129.74 38.8253) (width 0.25) (layer "B.Cu") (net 9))
 (segment (start 129.74 38.8253) (end 129.74 37.7) (width 0.25) (layer "B.Cu") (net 9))
 (segment (start 120.658 111.243) (end 128.99 102.911) (width 0.25) (layer "B.Cu") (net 9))
 (segment (start 137.36 45.32) (end 147.625 45.32) (width 0.25) (layer "B.Cu") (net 9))
 (segment (start 136.235 45.32) (end 136.235 45.0387) (width 0.25) (layer "B.Cu") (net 9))
 (segment (start 128.99 102.63) (end 130.115 102.63) (width 0.25) (layer "B.Cu") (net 9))
 (segment (start 128.99 102.911) (end 128.99 102.63) (width 0.25) (layer "B.Cu") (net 9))
 (segment (start 147.625 45.32) (end 151.815 49.51) (width 0.25) (layer "B.Cu") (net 9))
 (segment (start 101.19 109.6) (end 102.365 109.6) (width 0.25) (layer "B.Cu") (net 9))
 (segment (start 151.815 49.51) (end 152.94 49.51) (width 0.25) (layer "B.Cu") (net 9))
 (segment (start 103.641 111.243) (end 120.658 111.243) (width 0.25) (layer "B.Cu") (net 9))
 (segment (start 102.365 109.6) (end 102.365 109.967) (width 0.25) (layer "B.Cu") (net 9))
 (segment (start 137.36 45.32) (end 136.235 45.32) (width 0.25) (layer "B.Cu") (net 9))
 (segment (start 102.365 109.967) (end 103.641 111.243) (width 0.25) (layer "B.Cu") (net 9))
 (segment (start 136.235 45.0387) (end 130.021 38.8253) (width 0.25) (layer "B.Cu") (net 9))
 (segment (start 134.82 37.7) (end 134.82 38.8253) (width 0.25) (layer "F.Cu") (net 6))
 (segment (start 139.455 36.5747) (end 143.57 40.69) (width 0.25) (layer "F.Cu") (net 6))
 (segment (start 135.945 36.9966) (end 136.367 36.5747) (width 0.25) (layer "F.Cu") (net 6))
 (segment (start 129.26 49.4653) (end 129.26 49.51) (width 0.25) (layer "F.Cu") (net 6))
 (segment (start 134.82 37.7) (end 135.945 37.7) (width 0.25) (layer "F.Cu") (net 6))
 (segment (start 135.945 37.7) (end 135.945 36.9966) (width 0.25) (layer "F.Cu") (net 6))
 (segment (start 136.367 36.5747) (end 139.455 36.5747) (width 0.25) (layer "F.Cu") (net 6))
 (segment (start 132.28 41.3653) (end 132.28 45.32) (width 0.25) (layer "F.Cu") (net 6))
 (segment (start 132.28 45.32) (end 132.28 46.4453) (width 0.25) (layer "F.Cu") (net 6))
 (segment (start 134.82 38.8253) (end 132.28 41.3653) (width 0.25) (layer "F.Cu") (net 6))
 (segment (start 132.28 46.4453) (end 129.26 49.4653) (width 0.25) (layer "F.Cu") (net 6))
 (segment (start 115.2 39.42) (end 122.225 46.4454) (width 0.25) (layer "B.Cu") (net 6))
 (segment (start 122.225 46.4454) (end 126.195 46.4454) (width 0.25) (layer "B.Cu") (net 6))
 (segment (start 126.195 46.4454) (end 129.26 49.51) (width 0.25) (layer "B.Cu") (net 6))
 (segment (start 133.695 45.32) (end 133.695 45.0387) (width 0.25) (layer "B.Cu") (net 8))
 (segment (start 134.362 45.32) (end 133.695 45.32) (width 0.25) (layer "B.Cu") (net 8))
 (segment (start 134.362 45.32) (end 136.383 47.3411) (width 0.25) (layer "B.Cu") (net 8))
 (segment (start 128.076 39.42) (end 125.36 39.42) (width 0.25) (layer "B.Cu") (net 8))
 (segment (start 140.611 47.3411) (end 142.78 49.51) (width 0.25) (layer "B.Cu") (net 8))
 (segment (start 136.383 47.3411) (end 140.611 47.3411) (width 0.25) (layer "B.Cu") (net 8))
 (segment (start 133.695 45.0387) (end 128.076 39.42) (width 0.25) (layer "B.Cu") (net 8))
 (segment (start 134.82 45.32) (end 134.362 45.32) (width 0.25) (layer "B.Cu") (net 8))
 (segment (start 144.2297 53.1944) (end 140.5453 49.51) (width 0.25) (layer "F.Cu") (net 7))
 (segment (start 145.355 54.37) (end 144.2297 54.37) (width 0.25) (layer "F.Cu") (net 7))
 (segment (start 144.2297 54.37) (end 144.2297 53.1944) (width 0.25) (layer "F.Cu") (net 7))
 (segment (start 139.42 49.51) (end 140.5453 49.51) (width 0.25) (layer "F.Cu") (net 7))
 (segment (start 134.729 39.3047) (end 133.405 37.9814) (width 0.25) (layer "B.Cu") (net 11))
 (segment (start 156.609 39.3047) (end 134.729 39.3047) (width 0.25) (layer "B.Cu") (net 11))
 (segment (start 133.405 37.9814) (end 133.405 37.7) (width 0.25) (layer "B.Cu") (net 11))
 (segment (start 133.405 37.7) (end 132.28 37.7) (width 0.25) (layer "B.Cu") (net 11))
 (segment (start 159.46 40.73) (end 158.035 40.73) (width 0.25) (layer "B.Cu") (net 11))
 (segment (start 158.035 40.73) (end 156.609 39.3047) (width 0.25) (layer "B.Cu") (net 11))
 (segment (start 129.74 45.32) (end 130.865 45.32) (width 0.25) (layer "B.Cu") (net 13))
 (segment (start 130.865 45.6013) (end 135.955 50.6909) (width 0.25) (layer "B.Cu") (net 13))
 (segment (start 154.068 49.9848) (end 154.068 41.9678) (width 0.25) (layer "B.Cu") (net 13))
 (segment (start 135.955 50.6909) (end 153.362 50.6909) (width 0.25) (layer "B.Cu") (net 13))
 (segment (start 153.362 50.6909) (end 154.068 49.9848) (width 0.25) (layer "B.Cu") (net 13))
 (segment (start 130.865 45.32) (end 130.865 45.6013) (width 0.25) (layer "B.Cu") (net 13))
 (segment (start 154.068 41.9678) (end 152.79 40.69) (width 0.25) (layer "B.Cu") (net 13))
 (segment (start 159.46 48.35) (end 159.46 67.0797) (width 0.25) (layer "B.Cu") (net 10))
 (segment (start 125.035 101.505) (end 125.035 102.63) (width 0.25) (layer "B.Cu") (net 10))
 (segment (start 159.46 67.0797) (end 125.035 101.505) (width 0.25) (layer "B.Cu") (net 10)))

